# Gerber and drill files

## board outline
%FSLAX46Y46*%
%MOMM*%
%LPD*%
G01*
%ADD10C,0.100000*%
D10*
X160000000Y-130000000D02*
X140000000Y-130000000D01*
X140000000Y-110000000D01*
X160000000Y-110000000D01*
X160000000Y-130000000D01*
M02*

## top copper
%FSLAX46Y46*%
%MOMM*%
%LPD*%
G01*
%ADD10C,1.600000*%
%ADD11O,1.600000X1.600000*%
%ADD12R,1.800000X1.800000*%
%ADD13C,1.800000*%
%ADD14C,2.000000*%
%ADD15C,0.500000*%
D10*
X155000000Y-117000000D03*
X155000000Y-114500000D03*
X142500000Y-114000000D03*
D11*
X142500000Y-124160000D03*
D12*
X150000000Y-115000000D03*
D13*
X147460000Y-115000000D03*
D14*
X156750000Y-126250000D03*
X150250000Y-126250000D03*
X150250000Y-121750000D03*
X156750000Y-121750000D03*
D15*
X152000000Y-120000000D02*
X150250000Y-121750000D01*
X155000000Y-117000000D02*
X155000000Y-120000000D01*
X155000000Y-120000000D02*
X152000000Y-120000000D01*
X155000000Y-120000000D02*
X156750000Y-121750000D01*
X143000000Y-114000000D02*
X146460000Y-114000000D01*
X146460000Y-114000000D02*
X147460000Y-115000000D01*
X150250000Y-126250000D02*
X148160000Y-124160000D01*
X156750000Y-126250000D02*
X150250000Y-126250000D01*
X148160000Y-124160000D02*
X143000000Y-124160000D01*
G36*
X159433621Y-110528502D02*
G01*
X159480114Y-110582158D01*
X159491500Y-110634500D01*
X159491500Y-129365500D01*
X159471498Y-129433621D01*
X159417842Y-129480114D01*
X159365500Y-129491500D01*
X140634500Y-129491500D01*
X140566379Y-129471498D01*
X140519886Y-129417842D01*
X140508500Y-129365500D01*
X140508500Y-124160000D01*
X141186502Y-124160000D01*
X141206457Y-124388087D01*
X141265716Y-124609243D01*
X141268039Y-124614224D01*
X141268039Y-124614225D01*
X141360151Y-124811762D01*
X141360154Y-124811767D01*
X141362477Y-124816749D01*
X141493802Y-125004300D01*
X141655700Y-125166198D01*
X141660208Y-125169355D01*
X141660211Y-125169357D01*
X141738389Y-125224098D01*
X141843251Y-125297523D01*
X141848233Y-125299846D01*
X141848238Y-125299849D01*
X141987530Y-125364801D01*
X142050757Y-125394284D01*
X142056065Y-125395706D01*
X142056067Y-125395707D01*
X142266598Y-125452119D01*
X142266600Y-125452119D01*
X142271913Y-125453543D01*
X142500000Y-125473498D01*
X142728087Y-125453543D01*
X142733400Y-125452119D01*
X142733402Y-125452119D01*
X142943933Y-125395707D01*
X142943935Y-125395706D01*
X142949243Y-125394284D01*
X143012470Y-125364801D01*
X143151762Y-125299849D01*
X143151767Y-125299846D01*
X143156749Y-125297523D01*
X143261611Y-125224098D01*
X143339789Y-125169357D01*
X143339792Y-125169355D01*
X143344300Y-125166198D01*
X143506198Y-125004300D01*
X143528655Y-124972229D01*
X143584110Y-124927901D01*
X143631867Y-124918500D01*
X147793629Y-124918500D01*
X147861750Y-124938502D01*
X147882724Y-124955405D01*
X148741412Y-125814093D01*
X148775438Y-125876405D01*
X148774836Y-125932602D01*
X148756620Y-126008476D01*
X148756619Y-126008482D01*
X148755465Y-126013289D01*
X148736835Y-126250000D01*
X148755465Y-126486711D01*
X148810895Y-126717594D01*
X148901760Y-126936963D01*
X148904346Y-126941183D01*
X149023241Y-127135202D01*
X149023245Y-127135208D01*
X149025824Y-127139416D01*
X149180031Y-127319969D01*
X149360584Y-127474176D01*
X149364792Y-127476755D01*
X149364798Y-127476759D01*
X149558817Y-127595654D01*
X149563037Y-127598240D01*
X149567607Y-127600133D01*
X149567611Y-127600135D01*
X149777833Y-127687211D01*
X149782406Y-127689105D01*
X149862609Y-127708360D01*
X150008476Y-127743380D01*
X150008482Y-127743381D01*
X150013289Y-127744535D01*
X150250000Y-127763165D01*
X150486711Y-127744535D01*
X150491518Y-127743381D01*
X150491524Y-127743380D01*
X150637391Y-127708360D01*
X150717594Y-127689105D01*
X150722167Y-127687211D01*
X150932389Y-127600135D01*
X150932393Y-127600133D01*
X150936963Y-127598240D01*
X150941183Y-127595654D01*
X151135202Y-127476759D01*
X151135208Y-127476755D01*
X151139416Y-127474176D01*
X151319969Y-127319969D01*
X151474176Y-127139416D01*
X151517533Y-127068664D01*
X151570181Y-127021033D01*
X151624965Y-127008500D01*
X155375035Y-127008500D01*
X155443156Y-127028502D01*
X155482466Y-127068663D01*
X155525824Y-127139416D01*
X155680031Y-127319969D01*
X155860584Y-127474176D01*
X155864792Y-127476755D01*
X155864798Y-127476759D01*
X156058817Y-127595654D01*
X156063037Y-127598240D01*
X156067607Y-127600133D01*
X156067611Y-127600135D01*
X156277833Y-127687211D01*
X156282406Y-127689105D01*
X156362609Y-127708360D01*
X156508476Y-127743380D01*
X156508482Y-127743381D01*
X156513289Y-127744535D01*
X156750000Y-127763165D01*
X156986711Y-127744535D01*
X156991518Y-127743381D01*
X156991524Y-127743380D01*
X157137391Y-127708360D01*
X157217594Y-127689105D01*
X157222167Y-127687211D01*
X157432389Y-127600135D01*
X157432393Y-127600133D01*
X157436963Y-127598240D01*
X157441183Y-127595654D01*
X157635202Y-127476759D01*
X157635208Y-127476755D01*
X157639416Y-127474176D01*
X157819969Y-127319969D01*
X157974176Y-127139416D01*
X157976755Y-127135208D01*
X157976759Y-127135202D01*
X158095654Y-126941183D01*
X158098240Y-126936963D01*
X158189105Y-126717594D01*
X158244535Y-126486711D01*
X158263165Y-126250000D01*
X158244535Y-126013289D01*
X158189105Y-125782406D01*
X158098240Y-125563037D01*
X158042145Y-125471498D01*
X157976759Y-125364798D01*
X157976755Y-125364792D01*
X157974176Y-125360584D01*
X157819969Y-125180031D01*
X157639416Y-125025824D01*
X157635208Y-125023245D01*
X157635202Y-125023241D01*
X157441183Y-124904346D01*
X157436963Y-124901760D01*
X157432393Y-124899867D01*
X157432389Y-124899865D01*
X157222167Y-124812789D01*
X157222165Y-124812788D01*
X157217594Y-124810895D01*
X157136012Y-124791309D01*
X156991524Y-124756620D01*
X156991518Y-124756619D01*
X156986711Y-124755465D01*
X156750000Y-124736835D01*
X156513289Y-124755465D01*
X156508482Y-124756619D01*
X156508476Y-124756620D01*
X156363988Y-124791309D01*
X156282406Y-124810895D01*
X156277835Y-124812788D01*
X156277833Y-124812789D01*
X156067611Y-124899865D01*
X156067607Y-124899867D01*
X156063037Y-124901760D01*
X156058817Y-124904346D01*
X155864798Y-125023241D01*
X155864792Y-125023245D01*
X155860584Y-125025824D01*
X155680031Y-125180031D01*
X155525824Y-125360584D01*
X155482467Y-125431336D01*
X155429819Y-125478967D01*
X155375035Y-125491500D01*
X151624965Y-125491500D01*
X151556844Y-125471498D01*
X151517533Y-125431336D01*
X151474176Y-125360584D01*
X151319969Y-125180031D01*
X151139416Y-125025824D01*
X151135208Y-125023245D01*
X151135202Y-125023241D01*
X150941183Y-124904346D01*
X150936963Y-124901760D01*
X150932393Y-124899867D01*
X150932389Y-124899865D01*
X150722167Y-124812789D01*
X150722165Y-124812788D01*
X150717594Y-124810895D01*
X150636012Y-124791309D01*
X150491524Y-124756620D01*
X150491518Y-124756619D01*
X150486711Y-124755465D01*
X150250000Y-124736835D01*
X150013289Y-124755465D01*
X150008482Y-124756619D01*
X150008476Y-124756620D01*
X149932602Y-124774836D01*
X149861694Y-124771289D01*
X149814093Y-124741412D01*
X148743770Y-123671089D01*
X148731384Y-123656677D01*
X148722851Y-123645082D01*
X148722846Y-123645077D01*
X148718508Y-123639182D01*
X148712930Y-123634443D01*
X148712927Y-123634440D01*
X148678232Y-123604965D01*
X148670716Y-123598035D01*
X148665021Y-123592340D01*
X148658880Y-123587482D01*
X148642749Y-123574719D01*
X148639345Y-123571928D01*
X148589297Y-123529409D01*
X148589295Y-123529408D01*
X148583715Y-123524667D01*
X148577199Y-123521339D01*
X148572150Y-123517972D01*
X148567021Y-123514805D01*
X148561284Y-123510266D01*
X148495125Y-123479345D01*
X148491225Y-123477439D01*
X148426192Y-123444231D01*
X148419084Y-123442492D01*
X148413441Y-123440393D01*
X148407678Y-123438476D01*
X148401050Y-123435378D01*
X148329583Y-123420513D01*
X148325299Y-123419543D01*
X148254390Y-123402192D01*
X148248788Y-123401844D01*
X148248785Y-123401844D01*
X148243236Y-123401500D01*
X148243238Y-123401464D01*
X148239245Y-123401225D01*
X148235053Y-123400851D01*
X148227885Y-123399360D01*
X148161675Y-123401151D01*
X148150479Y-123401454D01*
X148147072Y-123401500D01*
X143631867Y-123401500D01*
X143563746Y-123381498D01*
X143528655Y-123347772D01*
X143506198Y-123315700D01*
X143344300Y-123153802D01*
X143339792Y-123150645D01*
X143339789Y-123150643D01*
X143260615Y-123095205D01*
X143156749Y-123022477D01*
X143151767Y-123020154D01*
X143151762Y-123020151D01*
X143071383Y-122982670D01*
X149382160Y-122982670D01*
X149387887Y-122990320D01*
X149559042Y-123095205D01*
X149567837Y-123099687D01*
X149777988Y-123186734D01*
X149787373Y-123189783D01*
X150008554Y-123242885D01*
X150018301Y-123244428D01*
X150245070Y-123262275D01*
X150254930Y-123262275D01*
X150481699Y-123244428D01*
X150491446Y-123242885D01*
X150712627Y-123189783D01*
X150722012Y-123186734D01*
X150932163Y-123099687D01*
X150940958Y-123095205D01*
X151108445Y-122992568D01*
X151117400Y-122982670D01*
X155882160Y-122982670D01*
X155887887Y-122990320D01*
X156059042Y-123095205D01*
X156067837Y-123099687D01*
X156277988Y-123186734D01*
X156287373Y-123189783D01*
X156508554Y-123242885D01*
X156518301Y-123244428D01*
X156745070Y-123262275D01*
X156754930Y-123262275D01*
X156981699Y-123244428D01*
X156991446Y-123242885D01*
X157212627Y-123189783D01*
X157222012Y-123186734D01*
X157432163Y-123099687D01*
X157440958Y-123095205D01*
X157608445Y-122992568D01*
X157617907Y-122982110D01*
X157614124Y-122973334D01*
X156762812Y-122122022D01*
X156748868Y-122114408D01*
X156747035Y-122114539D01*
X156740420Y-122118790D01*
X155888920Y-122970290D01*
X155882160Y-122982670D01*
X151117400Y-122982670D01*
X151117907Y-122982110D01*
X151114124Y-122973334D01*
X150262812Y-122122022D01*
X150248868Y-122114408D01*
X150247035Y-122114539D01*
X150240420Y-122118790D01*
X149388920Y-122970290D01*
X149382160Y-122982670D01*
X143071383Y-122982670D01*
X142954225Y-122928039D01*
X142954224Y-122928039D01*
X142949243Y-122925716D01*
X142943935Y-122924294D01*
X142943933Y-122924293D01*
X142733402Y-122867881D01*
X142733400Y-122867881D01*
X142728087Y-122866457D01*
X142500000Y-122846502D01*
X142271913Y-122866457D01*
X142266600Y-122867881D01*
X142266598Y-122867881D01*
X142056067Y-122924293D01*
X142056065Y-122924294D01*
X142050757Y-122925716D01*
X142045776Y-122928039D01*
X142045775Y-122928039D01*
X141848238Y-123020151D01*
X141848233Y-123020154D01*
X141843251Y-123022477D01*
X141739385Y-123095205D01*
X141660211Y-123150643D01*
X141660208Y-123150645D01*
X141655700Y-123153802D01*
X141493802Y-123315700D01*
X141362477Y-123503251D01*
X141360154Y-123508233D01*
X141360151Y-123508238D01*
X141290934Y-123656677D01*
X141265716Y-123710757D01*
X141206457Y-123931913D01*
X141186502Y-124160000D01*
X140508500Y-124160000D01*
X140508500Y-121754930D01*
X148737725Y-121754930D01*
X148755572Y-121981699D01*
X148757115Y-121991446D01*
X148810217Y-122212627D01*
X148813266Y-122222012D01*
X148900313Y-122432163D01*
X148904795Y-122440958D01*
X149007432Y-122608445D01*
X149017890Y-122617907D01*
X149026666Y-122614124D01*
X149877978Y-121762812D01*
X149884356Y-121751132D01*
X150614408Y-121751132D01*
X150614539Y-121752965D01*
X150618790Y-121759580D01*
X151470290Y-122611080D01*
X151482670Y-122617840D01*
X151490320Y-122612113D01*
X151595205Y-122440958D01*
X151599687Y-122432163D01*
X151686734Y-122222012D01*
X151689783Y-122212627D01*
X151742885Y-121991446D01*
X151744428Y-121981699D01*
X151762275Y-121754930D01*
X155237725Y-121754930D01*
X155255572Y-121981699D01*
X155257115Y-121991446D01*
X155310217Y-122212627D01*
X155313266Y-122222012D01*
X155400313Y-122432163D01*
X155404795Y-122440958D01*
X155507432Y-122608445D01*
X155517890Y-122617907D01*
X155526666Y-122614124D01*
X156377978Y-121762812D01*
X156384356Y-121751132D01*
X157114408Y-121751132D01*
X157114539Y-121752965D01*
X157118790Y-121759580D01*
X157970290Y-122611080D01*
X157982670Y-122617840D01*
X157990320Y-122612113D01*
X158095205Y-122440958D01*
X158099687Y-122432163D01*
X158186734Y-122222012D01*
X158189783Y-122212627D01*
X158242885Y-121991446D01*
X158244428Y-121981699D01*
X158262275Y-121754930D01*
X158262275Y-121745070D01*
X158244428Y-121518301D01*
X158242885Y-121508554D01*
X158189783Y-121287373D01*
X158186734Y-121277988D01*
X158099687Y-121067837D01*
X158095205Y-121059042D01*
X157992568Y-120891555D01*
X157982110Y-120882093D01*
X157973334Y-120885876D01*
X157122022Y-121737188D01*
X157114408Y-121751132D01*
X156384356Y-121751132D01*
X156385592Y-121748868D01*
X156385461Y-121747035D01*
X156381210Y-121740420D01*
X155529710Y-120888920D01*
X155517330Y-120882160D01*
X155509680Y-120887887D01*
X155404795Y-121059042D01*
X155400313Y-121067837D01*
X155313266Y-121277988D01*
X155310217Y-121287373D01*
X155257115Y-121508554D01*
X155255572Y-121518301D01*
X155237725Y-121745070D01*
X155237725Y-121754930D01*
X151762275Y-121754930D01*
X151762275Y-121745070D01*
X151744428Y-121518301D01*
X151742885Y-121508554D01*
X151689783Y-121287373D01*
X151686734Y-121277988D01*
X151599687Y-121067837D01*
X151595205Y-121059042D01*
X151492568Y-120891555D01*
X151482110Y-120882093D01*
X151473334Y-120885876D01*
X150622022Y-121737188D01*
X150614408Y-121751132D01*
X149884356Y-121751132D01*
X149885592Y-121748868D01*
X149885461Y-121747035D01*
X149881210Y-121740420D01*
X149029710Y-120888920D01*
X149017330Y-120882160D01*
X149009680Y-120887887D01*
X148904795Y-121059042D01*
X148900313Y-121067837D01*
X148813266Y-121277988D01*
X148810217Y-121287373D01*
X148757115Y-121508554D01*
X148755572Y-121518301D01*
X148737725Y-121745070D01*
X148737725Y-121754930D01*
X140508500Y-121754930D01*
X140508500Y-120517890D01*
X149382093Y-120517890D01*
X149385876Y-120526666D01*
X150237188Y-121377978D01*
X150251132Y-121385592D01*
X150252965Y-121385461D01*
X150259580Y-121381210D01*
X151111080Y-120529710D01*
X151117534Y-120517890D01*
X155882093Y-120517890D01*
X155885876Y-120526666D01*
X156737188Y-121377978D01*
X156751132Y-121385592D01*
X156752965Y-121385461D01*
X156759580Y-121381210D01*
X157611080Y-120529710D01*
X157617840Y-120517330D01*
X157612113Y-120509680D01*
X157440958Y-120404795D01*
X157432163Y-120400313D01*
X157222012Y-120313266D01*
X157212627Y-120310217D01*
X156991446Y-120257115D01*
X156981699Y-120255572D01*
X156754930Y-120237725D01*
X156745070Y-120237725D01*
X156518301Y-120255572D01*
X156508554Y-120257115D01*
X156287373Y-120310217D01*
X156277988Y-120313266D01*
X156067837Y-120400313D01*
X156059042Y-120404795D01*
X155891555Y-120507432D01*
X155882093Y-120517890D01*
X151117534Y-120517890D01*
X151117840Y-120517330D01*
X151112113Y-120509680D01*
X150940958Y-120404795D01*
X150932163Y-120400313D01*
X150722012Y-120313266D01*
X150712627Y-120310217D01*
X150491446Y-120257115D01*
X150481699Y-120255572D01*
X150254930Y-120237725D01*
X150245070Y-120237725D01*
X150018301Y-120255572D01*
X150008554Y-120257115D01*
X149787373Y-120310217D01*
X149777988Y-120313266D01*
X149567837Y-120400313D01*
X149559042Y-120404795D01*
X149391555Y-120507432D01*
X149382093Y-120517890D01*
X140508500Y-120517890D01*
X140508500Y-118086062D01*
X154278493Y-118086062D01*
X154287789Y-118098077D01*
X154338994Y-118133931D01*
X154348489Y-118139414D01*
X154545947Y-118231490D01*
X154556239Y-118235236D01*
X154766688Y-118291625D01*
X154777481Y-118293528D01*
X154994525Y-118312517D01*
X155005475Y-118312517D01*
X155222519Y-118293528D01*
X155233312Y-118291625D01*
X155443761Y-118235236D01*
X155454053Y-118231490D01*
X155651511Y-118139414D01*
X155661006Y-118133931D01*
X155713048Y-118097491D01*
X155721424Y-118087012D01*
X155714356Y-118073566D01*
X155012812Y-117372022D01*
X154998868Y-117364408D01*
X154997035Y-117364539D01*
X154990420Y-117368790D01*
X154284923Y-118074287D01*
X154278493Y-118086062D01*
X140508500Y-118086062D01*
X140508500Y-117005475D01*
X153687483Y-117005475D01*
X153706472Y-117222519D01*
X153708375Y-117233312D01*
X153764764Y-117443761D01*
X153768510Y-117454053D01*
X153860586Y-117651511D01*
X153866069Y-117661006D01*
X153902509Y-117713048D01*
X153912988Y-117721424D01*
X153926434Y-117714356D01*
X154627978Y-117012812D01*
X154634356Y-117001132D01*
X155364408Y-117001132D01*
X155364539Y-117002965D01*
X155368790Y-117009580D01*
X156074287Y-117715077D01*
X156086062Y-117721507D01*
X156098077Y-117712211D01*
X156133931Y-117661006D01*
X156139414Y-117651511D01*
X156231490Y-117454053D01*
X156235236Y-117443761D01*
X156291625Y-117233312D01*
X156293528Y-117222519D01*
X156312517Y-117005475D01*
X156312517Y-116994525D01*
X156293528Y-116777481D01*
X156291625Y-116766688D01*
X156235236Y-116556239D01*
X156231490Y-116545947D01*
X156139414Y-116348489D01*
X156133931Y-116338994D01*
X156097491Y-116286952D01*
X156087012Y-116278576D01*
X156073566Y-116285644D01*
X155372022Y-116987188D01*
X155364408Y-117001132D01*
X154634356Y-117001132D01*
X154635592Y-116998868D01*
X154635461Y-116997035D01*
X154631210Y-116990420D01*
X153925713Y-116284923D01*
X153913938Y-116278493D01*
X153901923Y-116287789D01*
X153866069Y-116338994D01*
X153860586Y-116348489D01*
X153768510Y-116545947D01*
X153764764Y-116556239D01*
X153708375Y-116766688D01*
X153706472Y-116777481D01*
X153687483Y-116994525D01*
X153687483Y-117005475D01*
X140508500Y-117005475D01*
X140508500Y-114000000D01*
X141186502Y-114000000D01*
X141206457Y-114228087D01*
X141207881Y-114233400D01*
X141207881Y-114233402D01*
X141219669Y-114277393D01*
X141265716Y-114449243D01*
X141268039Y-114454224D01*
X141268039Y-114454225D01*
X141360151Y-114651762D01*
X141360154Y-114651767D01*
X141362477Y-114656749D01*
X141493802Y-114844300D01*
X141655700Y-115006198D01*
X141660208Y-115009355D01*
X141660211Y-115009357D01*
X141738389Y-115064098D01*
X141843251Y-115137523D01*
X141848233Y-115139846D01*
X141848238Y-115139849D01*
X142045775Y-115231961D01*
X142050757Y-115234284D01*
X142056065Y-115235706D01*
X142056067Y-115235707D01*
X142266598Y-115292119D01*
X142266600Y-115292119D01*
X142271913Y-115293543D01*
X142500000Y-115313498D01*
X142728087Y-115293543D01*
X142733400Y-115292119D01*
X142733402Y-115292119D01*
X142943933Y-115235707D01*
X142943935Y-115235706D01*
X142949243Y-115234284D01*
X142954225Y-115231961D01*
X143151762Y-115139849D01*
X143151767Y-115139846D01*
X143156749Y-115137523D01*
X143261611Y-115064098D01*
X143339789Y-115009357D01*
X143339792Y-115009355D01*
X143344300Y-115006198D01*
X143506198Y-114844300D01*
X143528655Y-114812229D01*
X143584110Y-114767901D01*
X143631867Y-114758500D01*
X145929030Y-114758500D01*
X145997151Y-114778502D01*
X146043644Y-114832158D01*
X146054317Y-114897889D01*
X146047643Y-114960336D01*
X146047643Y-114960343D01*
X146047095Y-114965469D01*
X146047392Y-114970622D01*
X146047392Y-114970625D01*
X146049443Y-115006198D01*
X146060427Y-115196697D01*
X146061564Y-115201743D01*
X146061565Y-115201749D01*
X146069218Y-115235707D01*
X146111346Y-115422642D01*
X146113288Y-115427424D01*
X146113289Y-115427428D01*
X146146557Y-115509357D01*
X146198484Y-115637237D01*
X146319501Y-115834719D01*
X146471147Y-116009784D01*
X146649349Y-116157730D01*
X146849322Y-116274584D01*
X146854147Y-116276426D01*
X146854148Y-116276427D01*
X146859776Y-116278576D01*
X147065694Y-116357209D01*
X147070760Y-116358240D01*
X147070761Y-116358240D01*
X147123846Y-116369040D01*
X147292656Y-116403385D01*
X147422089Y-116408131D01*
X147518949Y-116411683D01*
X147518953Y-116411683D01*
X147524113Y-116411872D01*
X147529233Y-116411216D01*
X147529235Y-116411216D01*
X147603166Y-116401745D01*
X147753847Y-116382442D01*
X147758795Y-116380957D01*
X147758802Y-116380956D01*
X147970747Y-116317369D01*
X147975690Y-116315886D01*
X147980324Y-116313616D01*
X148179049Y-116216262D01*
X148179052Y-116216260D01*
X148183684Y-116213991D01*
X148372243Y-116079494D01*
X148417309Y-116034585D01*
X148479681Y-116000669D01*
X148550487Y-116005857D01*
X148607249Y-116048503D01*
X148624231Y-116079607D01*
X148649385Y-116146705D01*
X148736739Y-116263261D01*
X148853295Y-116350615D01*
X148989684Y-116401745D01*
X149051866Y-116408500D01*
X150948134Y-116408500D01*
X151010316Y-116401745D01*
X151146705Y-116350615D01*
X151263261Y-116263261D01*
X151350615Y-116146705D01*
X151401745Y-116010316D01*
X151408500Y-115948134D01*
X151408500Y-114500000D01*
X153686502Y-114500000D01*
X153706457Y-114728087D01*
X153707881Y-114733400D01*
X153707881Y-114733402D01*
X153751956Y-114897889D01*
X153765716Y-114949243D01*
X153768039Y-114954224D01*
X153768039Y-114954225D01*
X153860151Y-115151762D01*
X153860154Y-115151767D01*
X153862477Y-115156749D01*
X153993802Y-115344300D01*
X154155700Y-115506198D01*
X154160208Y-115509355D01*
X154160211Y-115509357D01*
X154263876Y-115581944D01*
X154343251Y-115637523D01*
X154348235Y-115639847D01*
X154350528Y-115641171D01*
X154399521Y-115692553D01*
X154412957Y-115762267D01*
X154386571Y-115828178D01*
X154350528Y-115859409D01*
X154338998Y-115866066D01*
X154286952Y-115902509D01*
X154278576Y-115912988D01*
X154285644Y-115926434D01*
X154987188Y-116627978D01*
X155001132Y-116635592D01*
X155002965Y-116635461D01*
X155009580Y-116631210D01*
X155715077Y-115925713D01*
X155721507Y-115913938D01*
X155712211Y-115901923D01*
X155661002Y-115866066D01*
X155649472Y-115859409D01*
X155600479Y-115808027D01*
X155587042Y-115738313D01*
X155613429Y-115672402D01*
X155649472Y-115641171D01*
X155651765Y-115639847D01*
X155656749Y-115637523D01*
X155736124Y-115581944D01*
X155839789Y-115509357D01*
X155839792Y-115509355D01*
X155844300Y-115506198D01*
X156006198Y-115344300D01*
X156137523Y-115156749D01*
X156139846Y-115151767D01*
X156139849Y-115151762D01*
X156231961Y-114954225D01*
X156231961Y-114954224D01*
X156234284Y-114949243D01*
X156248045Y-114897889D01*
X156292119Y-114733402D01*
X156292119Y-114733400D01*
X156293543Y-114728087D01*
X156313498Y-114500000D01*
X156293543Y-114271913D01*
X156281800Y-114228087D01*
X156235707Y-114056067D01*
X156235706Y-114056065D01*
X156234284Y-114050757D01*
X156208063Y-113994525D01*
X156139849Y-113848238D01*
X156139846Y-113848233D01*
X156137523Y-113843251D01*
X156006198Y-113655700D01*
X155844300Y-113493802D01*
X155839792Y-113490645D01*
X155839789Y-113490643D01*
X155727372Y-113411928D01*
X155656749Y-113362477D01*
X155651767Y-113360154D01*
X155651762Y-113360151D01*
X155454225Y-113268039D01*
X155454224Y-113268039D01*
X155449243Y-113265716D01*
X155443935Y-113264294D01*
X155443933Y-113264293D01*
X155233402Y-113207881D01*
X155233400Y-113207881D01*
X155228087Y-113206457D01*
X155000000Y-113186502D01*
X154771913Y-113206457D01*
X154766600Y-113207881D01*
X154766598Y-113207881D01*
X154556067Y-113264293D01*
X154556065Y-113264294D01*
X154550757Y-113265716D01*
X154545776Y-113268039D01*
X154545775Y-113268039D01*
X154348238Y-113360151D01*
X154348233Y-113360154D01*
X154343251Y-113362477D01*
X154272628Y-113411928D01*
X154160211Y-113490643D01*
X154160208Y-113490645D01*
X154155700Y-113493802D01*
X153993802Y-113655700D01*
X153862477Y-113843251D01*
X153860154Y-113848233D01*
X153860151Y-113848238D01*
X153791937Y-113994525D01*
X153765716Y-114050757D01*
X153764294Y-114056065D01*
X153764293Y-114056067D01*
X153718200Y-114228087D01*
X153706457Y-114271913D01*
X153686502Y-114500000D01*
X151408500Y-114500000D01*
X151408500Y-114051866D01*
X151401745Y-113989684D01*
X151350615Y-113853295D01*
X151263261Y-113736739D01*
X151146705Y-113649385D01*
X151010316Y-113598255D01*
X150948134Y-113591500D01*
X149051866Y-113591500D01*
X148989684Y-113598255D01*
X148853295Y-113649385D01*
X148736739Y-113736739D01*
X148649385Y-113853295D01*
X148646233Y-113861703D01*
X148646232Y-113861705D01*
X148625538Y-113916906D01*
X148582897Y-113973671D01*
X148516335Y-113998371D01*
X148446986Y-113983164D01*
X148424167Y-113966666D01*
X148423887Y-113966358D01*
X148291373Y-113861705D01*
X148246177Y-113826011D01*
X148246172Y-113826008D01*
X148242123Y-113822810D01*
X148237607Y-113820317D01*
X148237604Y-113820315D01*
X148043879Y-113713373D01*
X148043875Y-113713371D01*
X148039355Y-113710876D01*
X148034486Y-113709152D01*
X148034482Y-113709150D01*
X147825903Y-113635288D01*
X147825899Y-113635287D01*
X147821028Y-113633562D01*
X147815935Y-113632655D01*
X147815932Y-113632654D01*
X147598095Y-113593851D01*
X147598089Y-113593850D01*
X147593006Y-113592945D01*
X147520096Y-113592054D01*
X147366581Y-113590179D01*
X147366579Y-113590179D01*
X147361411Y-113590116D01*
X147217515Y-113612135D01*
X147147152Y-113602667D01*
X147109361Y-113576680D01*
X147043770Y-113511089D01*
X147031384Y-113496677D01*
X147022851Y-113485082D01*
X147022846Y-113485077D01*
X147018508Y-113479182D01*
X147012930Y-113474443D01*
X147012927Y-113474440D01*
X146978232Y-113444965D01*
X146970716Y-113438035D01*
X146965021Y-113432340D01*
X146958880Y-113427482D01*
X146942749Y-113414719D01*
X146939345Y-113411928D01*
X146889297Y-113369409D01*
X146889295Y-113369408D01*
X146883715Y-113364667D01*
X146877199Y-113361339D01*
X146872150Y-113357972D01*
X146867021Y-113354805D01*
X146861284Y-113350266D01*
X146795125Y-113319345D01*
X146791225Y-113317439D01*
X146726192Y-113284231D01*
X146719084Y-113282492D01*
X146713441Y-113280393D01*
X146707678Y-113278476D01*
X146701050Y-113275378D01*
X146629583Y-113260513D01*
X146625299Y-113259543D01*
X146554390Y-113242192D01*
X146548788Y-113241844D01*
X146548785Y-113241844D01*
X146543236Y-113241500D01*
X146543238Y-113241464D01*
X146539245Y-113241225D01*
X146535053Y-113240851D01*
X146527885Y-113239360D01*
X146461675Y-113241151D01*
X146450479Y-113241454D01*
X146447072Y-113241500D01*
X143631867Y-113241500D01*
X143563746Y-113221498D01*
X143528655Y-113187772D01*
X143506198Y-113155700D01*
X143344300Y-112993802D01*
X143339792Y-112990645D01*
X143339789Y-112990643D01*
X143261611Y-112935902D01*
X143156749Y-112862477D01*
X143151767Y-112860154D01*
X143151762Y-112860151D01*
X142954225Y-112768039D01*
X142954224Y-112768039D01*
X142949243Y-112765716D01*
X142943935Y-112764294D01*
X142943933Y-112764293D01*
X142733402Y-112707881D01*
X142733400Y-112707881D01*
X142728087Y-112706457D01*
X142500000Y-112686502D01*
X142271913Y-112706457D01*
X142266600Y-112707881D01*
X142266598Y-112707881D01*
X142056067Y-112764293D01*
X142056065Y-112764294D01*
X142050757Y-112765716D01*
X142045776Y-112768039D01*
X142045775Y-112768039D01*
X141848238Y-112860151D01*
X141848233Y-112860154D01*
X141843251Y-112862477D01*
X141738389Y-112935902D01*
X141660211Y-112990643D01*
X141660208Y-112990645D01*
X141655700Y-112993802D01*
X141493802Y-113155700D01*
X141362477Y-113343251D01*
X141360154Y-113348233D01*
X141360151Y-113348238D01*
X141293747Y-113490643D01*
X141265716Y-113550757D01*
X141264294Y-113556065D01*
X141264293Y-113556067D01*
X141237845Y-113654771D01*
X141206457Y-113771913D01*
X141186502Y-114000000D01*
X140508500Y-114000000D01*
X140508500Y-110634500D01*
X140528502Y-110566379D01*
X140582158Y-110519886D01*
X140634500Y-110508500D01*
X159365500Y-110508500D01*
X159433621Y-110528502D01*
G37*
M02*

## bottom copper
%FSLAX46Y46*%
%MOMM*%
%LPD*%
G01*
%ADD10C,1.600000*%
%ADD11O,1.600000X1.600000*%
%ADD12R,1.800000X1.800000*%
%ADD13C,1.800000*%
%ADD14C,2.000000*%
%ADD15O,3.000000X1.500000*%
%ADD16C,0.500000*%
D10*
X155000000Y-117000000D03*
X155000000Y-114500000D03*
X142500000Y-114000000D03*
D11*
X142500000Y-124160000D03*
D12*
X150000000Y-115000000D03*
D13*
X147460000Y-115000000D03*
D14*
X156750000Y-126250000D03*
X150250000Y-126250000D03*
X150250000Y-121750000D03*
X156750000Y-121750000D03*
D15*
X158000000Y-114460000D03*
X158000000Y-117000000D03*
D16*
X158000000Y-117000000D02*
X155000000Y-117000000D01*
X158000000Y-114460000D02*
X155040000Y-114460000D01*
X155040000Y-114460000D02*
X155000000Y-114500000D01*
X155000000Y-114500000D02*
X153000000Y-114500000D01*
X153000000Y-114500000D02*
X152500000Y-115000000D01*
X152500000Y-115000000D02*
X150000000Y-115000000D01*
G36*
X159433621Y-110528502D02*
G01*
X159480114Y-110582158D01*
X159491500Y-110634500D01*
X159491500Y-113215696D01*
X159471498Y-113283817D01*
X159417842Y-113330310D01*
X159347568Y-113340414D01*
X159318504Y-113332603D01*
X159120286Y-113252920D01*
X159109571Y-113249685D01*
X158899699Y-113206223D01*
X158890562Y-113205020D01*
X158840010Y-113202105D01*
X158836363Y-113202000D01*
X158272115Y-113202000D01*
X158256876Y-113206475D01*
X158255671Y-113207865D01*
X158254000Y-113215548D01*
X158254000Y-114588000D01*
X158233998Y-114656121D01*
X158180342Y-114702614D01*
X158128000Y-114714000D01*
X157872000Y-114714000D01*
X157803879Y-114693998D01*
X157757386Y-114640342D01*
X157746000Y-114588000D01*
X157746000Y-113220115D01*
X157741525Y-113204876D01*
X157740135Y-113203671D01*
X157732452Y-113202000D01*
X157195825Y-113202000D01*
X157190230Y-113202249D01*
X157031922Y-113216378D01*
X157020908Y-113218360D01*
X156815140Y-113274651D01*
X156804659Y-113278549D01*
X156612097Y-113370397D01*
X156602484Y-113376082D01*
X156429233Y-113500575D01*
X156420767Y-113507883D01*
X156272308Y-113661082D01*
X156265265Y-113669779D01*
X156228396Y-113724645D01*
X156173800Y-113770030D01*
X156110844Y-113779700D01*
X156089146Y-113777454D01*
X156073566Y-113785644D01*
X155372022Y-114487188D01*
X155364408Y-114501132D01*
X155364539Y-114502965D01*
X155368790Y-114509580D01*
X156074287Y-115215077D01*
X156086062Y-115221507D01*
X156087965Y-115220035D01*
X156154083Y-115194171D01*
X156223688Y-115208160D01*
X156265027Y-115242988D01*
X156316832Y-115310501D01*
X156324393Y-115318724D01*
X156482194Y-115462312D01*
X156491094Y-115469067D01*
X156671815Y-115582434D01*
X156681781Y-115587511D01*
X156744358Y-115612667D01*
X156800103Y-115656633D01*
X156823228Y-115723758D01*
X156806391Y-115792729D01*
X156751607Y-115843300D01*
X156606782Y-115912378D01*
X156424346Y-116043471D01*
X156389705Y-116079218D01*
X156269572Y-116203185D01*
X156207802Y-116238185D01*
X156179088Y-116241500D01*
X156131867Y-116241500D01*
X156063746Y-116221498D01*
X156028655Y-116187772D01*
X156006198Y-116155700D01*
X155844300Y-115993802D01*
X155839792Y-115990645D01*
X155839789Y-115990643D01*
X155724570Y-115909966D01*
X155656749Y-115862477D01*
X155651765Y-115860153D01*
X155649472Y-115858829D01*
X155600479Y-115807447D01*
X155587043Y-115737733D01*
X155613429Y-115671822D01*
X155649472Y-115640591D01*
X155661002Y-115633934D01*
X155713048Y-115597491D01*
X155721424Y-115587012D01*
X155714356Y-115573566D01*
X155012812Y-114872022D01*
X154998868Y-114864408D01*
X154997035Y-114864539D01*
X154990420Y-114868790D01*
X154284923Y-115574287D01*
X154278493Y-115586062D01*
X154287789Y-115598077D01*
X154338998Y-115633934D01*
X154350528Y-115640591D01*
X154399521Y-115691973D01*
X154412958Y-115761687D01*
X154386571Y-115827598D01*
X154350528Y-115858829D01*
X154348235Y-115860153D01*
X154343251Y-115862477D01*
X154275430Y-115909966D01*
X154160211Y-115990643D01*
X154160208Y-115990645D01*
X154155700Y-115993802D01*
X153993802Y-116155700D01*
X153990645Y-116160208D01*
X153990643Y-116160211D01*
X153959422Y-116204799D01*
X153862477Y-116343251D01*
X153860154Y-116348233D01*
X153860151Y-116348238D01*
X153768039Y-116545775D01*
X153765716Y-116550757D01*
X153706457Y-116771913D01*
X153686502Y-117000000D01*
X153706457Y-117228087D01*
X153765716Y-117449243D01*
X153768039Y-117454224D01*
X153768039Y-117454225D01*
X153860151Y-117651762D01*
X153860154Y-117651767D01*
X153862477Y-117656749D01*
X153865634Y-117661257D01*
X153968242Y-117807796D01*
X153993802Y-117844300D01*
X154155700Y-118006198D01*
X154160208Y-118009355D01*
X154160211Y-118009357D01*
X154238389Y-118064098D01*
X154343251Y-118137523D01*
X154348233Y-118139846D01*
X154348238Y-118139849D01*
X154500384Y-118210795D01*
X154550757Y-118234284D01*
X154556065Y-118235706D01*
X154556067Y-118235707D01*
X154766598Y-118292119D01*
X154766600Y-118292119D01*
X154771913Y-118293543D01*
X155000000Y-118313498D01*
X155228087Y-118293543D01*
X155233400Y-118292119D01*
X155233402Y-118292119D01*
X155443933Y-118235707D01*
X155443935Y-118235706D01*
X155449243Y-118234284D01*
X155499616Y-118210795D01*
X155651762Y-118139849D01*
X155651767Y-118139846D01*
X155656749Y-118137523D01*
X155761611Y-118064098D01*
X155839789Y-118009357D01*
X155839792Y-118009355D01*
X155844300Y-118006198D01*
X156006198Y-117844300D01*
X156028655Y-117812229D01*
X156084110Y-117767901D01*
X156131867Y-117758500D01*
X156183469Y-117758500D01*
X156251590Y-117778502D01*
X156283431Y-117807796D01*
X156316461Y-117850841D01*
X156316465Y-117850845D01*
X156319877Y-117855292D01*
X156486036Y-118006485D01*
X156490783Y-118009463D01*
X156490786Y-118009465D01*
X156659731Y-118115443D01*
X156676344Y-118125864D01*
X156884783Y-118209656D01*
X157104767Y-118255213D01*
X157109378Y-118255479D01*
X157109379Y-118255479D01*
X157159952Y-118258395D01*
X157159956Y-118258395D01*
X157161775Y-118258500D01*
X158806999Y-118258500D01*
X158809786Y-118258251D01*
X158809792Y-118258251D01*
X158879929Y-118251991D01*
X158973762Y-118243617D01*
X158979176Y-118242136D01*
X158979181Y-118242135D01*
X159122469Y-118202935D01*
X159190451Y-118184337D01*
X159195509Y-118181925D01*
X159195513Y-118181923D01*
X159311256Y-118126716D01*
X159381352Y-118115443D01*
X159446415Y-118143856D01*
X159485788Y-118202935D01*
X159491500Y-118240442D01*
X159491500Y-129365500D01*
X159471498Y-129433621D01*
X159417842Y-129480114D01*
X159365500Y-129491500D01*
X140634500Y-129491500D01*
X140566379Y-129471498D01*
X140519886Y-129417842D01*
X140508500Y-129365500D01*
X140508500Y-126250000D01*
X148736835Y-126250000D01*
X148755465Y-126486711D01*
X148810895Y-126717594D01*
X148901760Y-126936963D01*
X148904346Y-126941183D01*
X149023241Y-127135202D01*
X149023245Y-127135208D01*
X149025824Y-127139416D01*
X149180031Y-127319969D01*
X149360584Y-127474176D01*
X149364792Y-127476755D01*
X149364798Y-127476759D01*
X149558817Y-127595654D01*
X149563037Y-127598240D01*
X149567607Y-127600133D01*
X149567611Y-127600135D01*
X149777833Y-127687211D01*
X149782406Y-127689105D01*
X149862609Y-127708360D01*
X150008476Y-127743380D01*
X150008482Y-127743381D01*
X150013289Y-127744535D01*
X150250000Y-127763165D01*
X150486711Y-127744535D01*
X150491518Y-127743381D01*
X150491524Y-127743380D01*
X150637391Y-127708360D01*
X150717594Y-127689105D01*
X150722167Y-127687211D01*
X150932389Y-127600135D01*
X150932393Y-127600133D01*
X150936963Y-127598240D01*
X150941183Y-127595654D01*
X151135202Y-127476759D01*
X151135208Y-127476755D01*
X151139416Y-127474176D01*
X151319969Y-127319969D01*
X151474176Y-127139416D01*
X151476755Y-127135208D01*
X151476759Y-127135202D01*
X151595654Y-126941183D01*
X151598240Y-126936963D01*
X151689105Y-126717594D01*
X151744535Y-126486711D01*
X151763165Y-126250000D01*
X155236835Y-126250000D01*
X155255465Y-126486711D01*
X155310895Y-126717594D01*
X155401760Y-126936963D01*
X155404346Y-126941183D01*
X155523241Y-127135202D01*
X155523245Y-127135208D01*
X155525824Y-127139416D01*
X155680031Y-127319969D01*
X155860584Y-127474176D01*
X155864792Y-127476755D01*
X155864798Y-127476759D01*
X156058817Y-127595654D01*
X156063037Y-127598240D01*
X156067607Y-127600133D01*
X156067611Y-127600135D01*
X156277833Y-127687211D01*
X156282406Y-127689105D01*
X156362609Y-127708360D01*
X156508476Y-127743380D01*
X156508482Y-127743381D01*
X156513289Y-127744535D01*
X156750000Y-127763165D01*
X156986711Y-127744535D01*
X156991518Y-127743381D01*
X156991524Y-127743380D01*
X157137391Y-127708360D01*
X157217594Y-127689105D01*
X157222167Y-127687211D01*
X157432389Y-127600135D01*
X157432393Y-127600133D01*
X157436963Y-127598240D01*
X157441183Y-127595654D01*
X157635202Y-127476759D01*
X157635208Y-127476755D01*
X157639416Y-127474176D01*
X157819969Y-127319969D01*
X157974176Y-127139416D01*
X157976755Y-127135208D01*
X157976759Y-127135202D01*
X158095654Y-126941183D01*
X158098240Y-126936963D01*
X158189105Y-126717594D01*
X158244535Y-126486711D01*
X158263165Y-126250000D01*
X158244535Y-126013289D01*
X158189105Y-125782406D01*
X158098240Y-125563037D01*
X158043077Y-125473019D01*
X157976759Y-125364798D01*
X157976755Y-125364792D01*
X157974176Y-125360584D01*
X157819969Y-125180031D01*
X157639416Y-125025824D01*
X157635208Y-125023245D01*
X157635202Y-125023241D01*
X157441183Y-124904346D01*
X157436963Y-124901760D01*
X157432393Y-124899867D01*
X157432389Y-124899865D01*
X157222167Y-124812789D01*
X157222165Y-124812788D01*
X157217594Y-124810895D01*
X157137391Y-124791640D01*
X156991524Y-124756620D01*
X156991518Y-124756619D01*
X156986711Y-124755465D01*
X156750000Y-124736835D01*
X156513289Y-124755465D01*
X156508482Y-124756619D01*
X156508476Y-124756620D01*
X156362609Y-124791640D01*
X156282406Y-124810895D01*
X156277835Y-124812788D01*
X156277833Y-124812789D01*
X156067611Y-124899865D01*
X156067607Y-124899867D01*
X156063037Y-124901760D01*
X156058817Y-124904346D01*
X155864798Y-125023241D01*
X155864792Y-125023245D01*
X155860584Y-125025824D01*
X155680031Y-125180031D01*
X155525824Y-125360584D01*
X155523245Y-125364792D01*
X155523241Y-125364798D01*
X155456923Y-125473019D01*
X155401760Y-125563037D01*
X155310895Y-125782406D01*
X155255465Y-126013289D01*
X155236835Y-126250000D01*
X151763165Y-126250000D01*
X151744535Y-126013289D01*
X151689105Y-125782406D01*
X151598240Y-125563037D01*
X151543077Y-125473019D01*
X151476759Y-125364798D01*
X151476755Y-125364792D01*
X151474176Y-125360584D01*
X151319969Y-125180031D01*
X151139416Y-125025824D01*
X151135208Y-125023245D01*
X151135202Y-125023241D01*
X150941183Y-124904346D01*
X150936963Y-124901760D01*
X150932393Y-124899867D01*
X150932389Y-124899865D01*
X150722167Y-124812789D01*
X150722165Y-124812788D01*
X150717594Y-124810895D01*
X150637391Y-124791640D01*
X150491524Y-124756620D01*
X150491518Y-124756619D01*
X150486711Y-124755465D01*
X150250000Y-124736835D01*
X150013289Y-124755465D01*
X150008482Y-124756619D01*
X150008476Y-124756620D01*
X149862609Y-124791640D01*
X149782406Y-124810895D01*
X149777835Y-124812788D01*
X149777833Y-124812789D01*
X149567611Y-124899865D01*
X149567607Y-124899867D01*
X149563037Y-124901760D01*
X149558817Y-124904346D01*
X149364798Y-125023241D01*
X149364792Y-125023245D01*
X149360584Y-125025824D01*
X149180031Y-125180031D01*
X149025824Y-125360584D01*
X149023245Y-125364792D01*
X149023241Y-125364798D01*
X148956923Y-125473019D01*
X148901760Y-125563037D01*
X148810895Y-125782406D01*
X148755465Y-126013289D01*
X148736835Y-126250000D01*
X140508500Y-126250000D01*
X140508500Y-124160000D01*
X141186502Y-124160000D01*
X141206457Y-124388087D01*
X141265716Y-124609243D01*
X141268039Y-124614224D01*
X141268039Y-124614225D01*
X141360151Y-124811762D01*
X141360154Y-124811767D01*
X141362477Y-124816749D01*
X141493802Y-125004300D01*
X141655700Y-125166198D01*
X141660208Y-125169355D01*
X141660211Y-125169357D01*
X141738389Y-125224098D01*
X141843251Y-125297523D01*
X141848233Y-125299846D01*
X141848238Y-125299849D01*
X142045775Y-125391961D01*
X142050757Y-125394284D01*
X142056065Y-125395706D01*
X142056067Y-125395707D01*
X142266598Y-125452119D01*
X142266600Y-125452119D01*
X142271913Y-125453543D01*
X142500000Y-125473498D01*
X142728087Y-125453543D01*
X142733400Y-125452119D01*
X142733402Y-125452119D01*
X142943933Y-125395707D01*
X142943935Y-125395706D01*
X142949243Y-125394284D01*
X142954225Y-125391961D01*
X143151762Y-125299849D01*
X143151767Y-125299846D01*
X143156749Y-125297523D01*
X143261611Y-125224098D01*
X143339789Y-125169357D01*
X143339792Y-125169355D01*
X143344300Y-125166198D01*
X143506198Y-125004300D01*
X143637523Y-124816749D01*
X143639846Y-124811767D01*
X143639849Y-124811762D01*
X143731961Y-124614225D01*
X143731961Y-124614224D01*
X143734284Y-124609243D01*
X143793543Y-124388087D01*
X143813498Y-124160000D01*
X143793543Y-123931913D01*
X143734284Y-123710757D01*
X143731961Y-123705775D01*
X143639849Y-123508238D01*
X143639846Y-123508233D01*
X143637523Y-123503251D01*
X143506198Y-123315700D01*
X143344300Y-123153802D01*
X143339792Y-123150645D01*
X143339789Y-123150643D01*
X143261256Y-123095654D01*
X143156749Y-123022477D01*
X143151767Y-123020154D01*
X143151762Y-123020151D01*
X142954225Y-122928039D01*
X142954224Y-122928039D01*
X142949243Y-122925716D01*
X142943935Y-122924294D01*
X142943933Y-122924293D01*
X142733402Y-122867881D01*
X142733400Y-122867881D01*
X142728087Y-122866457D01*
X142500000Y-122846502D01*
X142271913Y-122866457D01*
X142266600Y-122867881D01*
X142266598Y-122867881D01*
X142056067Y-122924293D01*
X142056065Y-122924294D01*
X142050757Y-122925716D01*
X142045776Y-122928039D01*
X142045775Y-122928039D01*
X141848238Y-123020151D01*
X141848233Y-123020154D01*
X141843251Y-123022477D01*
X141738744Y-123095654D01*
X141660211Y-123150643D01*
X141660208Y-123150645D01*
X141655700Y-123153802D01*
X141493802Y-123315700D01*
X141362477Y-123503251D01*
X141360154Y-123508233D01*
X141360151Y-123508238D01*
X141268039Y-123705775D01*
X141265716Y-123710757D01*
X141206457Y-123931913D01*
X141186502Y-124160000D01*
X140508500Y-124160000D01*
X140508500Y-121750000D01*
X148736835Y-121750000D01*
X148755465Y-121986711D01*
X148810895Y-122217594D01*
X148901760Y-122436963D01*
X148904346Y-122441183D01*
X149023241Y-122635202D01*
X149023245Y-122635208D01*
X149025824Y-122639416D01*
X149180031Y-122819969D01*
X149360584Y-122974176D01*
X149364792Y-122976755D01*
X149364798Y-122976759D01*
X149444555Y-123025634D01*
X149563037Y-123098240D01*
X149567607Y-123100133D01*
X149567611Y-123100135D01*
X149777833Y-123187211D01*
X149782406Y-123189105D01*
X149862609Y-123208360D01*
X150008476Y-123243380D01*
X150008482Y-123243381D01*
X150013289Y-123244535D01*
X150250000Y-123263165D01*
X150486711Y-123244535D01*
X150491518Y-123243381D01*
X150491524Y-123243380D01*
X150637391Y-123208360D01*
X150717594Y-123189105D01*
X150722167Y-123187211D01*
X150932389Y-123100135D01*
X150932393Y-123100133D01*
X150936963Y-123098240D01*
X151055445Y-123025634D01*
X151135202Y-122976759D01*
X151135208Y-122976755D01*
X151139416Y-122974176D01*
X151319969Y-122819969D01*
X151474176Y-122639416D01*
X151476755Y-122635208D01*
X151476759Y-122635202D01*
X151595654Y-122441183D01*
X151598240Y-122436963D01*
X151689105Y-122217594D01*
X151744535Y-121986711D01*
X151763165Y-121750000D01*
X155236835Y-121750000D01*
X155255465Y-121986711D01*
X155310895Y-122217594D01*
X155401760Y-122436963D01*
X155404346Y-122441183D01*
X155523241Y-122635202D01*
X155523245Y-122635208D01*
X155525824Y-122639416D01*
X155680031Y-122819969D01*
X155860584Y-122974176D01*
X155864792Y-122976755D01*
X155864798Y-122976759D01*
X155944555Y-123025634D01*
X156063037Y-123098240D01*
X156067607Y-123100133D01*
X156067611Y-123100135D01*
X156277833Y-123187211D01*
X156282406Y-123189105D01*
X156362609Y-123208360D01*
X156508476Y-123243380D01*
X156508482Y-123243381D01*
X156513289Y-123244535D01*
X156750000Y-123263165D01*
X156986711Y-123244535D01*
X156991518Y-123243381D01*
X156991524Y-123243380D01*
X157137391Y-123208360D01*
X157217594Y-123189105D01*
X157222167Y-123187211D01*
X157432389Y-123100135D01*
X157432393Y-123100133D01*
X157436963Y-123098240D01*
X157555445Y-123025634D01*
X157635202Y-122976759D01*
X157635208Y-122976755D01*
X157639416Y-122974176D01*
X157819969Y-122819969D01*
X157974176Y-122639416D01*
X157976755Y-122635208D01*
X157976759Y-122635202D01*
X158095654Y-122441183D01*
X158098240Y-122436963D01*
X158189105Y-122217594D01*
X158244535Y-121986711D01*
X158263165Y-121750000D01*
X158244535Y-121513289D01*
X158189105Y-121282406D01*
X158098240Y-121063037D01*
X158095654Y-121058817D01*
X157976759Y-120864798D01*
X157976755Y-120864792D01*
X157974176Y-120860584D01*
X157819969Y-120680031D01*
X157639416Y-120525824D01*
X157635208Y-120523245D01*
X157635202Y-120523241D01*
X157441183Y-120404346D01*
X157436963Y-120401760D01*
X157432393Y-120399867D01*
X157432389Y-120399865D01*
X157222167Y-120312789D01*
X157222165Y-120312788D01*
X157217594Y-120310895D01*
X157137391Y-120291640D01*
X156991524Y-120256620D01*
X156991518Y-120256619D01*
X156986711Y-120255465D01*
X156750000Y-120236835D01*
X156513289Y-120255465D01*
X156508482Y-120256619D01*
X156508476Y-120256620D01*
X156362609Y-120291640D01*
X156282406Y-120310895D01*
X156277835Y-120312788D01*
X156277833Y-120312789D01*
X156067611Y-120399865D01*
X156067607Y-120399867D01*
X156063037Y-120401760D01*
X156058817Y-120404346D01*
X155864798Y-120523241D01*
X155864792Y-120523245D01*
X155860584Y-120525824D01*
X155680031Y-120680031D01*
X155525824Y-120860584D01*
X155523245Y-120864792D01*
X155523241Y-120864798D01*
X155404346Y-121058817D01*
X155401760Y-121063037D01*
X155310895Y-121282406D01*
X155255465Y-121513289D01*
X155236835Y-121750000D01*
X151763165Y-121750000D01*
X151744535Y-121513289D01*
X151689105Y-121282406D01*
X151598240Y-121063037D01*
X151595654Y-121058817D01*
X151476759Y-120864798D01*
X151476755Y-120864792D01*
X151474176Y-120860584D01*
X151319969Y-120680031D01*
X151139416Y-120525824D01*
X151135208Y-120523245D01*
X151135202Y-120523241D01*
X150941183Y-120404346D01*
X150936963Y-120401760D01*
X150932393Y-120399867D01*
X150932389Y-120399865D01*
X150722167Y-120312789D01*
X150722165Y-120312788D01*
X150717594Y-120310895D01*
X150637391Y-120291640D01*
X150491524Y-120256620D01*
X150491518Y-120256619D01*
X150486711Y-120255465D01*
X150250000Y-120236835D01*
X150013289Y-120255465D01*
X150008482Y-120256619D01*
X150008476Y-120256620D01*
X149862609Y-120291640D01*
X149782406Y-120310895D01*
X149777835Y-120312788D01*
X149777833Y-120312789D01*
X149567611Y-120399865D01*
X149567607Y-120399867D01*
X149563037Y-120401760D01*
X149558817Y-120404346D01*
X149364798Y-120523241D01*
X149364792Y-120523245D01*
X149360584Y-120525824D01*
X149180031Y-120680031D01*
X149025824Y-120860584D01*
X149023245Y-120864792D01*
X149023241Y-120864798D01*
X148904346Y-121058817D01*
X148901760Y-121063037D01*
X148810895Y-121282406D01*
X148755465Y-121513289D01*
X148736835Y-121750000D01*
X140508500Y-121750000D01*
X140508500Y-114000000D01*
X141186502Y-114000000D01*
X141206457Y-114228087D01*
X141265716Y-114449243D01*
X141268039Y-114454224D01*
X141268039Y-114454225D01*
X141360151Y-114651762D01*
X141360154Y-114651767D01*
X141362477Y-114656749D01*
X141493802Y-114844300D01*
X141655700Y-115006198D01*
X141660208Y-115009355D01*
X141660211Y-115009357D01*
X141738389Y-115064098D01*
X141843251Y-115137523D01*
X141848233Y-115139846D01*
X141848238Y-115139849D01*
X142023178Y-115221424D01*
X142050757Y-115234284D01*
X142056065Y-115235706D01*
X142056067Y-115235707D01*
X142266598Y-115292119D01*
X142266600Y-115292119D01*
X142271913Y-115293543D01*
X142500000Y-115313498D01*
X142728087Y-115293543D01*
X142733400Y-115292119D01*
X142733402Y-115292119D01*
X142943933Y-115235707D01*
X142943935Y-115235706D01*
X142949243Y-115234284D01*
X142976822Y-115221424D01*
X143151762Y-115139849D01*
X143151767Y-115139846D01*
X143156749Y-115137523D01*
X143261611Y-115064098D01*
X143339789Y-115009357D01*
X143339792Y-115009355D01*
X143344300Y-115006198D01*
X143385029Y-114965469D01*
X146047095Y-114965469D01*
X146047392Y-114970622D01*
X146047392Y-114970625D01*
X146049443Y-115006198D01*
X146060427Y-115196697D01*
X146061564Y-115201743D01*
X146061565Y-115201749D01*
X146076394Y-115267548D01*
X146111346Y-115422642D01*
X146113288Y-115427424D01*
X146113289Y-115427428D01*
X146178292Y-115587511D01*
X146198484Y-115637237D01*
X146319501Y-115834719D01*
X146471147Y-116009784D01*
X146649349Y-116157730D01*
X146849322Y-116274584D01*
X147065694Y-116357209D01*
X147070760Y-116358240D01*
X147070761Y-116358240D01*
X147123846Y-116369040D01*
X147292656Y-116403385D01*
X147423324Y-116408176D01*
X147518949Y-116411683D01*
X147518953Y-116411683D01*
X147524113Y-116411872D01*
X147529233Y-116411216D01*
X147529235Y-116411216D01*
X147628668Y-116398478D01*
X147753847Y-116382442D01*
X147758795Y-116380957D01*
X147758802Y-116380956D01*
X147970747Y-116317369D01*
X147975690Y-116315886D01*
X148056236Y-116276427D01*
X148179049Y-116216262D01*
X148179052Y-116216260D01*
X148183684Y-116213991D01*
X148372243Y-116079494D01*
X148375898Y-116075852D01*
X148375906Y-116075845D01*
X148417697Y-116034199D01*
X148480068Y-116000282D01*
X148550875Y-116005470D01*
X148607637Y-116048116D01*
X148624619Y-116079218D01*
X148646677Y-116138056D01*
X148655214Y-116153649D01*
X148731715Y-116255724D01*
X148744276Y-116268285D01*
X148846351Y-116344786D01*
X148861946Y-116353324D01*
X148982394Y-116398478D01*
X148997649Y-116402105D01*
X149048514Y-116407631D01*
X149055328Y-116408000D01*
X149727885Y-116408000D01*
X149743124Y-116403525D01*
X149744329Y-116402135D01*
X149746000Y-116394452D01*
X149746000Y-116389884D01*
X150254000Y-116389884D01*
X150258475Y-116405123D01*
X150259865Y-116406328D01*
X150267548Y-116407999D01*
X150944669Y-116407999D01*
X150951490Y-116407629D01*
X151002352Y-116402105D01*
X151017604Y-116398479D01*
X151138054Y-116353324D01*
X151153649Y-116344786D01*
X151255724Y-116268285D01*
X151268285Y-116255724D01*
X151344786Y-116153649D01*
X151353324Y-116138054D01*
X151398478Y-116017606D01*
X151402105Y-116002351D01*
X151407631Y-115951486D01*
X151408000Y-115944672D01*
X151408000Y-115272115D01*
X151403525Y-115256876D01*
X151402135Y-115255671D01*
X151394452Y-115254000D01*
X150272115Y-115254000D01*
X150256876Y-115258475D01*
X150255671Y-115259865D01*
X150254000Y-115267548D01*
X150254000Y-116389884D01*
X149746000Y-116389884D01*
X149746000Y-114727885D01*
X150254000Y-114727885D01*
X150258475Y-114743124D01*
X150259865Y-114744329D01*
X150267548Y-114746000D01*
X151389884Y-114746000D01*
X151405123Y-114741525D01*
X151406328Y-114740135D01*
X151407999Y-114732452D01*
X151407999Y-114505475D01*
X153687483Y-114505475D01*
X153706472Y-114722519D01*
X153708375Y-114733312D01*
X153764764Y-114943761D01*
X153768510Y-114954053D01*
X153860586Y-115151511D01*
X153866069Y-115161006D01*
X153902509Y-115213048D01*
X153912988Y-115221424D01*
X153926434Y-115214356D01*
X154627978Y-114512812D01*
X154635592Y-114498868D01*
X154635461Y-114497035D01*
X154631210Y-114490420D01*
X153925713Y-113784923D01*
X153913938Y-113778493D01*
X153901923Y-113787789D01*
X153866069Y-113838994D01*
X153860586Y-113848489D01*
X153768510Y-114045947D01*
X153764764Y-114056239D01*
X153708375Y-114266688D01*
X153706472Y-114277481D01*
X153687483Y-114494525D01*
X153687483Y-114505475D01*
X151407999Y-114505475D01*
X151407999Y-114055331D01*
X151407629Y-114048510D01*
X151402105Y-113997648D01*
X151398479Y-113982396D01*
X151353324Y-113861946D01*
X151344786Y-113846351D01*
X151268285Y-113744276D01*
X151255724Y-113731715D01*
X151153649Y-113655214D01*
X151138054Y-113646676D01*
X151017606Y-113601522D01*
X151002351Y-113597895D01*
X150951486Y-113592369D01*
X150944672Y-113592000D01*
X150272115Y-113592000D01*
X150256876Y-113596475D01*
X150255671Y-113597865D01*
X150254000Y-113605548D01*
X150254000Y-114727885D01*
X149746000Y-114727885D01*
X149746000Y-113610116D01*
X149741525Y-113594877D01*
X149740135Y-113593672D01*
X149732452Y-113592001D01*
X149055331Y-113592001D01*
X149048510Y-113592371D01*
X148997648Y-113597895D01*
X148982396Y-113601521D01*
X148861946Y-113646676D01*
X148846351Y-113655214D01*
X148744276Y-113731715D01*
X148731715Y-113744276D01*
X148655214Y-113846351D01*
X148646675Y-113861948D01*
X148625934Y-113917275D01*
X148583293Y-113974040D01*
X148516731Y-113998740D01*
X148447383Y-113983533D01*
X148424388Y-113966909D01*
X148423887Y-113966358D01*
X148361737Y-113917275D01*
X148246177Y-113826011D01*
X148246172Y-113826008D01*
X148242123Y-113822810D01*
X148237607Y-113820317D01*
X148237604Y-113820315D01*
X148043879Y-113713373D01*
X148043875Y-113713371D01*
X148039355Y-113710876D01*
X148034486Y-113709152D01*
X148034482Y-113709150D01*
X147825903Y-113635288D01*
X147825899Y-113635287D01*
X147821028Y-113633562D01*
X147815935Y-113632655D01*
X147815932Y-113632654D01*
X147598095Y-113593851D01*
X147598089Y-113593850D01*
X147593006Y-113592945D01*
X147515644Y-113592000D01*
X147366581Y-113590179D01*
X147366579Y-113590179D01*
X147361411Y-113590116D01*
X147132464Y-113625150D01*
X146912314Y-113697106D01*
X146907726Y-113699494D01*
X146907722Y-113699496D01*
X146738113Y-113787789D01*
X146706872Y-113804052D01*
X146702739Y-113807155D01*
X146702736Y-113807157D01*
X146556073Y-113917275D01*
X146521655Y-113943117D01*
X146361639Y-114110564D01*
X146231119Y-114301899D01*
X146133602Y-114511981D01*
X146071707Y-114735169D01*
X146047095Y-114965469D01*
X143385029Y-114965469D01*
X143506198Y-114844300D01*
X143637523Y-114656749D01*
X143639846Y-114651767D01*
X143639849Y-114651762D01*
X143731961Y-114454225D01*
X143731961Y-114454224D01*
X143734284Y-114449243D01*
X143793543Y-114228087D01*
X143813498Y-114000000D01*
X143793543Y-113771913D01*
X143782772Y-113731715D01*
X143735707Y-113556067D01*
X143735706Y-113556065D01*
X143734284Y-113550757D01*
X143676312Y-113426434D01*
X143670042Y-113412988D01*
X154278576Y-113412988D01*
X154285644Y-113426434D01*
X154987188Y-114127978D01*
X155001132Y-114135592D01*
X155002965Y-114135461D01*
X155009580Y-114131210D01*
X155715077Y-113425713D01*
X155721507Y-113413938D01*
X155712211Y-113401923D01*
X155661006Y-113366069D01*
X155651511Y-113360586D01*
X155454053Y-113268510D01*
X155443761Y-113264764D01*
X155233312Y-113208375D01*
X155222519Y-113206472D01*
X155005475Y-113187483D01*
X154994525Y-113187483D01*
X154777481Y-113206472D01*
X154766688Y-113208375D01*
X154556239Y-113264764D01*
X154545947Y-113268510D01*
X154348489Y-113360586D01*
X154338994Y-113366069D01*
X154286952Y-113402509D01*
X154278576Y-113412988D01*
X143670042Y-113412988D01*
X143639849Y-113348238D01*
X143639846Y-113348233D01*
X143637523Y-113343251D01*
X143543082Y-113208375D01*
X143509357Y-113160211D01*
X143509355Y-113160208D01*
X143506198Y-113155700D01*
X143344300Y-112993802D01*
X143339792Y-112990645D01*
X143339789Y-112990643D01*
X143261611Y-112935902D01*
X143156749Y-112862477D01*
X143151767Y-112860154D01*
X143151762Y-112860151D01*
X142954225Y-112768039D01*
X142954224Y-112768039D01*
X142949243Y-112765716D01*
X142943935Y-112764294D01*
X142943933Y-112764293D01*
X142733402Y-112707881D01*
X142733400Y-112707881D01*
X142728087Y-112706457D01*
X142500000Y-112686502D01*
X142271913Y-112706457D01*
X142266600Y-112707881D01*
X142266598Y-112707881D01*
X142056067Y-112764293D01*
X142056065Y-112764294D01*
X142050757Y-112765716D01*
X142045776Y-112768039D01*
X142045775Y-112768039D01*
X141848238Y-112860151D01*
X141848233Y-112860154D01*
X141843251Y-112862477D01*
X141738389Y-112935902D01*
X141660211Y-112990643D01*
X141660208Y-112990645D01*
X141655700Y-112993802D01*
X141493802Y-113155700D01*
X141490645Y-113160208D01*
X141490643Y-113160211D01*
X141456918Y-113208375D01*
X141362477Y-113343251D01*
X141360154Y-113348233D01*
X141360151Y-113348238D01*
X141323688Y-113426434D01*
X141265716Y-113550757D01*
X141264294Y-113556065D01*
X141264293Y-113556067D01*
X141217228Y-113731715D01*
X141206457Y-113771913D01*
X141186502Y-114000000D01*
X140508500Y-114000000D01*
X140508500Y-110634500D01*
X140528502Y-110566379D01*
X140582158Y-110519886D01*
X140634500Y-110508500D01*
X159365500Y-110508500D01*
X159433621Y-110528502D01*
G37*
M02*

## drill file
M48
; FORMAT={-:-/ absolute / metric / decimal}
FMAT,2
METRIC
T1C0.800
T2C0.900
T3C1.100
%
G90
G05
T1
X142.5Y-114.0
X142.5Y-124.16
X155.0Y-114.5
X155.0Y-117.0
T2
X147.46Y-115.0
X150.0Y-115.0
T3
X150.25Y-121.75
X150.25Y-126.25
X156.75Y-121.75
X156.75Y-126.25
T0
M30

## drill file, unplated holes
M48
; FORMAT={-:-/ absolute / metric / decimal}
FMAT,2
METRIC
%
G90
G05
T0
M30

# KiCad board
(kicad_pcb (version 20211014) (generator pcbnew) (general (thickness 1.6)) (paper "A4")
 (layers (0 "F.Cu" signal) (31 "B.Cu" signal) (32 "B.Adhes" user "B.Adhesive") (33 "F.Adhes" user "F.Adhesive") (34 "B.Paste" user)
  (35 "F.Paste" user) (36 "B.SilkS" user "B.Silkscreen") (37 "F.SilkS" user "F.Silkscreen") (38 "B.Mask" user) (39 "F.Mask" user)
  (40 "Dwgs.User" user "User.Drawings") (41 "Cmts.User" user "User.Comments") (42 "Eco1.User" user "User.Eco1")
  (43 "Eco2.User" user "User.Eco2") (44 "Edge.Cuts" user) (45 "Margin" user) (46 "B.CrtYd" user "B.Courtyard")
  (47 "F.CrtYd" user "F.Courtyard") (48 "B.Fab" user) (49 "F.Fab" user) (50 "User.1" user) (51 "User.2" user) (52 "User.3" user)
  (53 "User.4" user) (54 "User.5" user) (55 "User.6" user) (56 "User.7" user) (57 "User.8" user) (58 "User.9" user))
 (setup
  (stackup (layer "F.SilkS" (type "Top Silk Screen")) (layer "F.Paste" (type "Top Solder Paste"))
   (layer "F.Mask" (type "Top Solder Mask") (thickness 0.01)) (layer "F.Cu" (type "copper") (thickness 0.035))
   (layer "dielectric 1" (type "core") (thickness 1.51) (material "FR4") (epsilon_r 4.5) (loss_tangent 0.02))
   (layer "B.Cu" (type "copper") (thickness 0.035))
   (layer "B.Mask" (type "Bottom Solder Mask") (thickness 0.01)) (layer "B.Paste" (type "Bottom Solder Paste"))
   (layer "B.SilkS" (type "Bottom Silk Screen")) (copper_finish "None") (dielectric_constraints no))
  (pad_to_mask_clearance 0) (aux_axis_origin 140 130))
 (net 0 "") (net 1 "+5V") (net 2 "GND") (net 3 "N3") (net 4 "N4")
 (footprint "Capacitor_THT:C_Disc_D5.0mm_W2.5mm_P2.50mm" (layer "F.Cu") (at 155 117 90)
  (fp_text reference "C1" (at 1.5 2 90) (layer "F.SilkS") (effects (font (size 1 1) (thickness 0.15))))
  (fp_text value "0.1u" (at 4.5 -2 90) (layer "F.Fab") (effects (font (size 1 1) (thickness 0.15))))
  (pad "1" thru_hole circle (at 0 0 90) (size 1.6 1.6) (drill 0.8) (layers *.Cu *.Mask) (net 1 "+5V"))
  (pad "2" thru_hole circle (at 2.5 0 90) (size 1.6 1.6) (drill 0.8) (layers *.Cu *.Mask) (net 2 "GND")))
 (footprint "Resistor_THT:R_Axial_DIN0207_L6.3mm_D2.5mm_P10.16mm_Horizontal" (layer "F.Cu") (at 142.5 114 -90)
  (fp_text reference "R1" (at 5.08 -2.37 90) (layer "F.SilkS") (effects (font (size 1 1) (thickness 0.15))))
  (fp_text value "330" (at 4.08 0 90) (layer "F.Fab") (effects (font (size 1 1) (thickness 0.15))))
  (pad "1" thru_hole circle (at 0 0 270) (size 1.6 1.6) (drill 0.8) (layers *.Cu *.Mask) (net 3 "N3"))
  (pad "2" thru_hole oval (at 10.16 0 270) (size 1.6 1.6) (drill 0.8) (layers *.Cu *.Mask) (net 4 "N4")))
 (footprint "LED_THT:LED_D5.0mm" (layer "F.Cu") (at 150 115 180)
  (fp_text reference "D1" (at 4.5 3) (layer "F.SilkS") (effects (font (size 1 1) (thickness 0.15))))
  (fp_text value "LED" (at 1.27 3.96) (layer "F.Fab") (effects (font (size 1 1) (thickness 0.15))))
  (pad "1" thru_hole rect (at 0 0 180) (size 1.8 1.8) (drill 0.9) (layers *.Cu *.Mask) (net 2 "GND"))
  (pad "2" thru_hole circle (at 2.54 0 180) (size 1.8 1.8) (drill 0.9) (layers *.Cu *.Mask) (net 3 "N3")))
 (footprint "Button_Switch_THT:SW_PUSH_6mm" (layer "F.Cu") (at 156.75 126.25 180)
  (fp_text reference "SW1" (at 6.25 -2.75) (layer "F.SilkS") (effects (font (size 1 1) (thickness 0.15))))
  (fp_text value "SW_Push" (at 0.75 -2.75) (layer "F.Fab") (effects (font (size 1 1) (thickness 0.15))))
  (pad "1" thru_hole circle (at 0 0 270) (size 2 2) (drill 1.1) (layers *.Cu *.Mask) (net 4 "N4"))
  (pad "1" thru_hole circle (at 6.5 0 270) (size 2 2) (drill 1.1) (layers *.Cu *.Mask) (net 4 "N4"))
  (pad "2" thru_hole circle (at 6.5 4.5 270) (size 2 2) (drill 1.1) (layers *.Cu *.Mask) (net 1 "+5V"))
  (pad "2" thru_hole circle (at 0 4.5 270) (size 2 2) (drill 1.1) (layers *.Cu *.Mask) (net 1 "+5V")))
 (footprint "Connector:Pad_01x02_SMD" (layer "B.Cu") (at 158 117)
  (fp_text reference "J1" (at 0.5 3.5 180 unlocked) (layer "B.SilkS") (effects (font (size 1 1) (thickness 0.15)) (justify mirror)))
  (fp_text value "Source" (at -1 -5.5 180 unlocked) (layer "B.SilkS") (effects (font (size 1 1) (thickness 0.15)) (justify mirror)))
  (pad "1" smd oval (at 0 -2.54 270) (size 1.5 3) (layers "B.Cu" "B.Paste" "B.Mask") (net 2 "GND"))
  (pad "2" smd oval (at 0 0 270) (size 1.5 3) (layers "B.Cu" "B.Paste" "B.Mask") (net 1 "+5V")))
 (gr_poly (pts (xy 160 130) (xy 140 130) (xy 140 110) (xy 160 110)) (layer "Edge.Cuts") (width 0.1) (fill none))
 (segment (start 152 120) (end 150.25 121.75) (width 0.5) (layer "F.Cu") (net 1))
 (segment (start 155 117) (end 155 120) (width 0.5) (layer "F.Cu") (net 1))
 (segment (start 155 120) (end 152 120) (width 0.5) (layer "F.Cu") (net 1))
 (segment (start 155 120) (end 156.75 121.75) (width 0.5) (layer "F.Cu") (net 1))
 (segment (start 158 117) (end 155 117) (width 0.5) (layer "B.Cu") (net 1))
 (segment (start 158 114.46) (end 155.04 114.46) (width 0.5) (layer "B.Cu") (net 2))
 (segment (start 155.04 114.46) (end 155 114.5) (width 0.5) (layer "B.Cu") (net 2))
 (segment (start 155 114.5) (end 153 114.5) (width 0.5) (layer "B.Cu") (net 2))
 (segment (start 153 114.5) (end 152.5 115) (width 0.5) (layer "B.Cu") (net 2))
 (segment (start 152.5 115) (end 150 115) (width 0.5) (layer "B.Cu") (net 2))
 (segment (start 143 114) (end 146.46 114) (width 0.5) (layer "F.Cu") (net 3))
 (segment (start 146.46 114) (end 147.46 115) (width 0.5) (layer "F.Cu") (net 3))
 (segment (start 150.25 126.25) (end 148.16 124.16) (width 0.5) (layer "F.Cu") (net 4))
 (segment (start 156.75 126.25) (end 150.25 126.25) (width 0.5) (layer "F.Cu") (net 4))
 (segment (start 148.16 124.16) (end 143 124.16) (width 0.5) (layer "F.Cu") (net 4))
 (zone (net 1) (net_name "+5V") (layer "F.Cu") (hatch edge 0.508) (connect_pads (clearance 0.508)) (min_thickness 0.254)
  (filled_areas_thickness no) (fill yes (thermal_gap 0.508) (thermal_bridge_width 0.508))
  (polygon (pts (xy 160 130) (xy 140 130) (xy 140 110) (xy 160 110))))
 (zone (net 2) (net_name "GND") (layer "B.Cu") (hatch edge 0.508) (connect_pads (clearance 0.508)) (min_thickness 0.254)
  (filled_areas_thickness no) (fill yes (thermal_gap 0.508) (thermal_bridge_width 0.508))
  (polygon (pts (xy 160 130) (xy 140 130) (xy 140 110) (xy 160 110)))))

